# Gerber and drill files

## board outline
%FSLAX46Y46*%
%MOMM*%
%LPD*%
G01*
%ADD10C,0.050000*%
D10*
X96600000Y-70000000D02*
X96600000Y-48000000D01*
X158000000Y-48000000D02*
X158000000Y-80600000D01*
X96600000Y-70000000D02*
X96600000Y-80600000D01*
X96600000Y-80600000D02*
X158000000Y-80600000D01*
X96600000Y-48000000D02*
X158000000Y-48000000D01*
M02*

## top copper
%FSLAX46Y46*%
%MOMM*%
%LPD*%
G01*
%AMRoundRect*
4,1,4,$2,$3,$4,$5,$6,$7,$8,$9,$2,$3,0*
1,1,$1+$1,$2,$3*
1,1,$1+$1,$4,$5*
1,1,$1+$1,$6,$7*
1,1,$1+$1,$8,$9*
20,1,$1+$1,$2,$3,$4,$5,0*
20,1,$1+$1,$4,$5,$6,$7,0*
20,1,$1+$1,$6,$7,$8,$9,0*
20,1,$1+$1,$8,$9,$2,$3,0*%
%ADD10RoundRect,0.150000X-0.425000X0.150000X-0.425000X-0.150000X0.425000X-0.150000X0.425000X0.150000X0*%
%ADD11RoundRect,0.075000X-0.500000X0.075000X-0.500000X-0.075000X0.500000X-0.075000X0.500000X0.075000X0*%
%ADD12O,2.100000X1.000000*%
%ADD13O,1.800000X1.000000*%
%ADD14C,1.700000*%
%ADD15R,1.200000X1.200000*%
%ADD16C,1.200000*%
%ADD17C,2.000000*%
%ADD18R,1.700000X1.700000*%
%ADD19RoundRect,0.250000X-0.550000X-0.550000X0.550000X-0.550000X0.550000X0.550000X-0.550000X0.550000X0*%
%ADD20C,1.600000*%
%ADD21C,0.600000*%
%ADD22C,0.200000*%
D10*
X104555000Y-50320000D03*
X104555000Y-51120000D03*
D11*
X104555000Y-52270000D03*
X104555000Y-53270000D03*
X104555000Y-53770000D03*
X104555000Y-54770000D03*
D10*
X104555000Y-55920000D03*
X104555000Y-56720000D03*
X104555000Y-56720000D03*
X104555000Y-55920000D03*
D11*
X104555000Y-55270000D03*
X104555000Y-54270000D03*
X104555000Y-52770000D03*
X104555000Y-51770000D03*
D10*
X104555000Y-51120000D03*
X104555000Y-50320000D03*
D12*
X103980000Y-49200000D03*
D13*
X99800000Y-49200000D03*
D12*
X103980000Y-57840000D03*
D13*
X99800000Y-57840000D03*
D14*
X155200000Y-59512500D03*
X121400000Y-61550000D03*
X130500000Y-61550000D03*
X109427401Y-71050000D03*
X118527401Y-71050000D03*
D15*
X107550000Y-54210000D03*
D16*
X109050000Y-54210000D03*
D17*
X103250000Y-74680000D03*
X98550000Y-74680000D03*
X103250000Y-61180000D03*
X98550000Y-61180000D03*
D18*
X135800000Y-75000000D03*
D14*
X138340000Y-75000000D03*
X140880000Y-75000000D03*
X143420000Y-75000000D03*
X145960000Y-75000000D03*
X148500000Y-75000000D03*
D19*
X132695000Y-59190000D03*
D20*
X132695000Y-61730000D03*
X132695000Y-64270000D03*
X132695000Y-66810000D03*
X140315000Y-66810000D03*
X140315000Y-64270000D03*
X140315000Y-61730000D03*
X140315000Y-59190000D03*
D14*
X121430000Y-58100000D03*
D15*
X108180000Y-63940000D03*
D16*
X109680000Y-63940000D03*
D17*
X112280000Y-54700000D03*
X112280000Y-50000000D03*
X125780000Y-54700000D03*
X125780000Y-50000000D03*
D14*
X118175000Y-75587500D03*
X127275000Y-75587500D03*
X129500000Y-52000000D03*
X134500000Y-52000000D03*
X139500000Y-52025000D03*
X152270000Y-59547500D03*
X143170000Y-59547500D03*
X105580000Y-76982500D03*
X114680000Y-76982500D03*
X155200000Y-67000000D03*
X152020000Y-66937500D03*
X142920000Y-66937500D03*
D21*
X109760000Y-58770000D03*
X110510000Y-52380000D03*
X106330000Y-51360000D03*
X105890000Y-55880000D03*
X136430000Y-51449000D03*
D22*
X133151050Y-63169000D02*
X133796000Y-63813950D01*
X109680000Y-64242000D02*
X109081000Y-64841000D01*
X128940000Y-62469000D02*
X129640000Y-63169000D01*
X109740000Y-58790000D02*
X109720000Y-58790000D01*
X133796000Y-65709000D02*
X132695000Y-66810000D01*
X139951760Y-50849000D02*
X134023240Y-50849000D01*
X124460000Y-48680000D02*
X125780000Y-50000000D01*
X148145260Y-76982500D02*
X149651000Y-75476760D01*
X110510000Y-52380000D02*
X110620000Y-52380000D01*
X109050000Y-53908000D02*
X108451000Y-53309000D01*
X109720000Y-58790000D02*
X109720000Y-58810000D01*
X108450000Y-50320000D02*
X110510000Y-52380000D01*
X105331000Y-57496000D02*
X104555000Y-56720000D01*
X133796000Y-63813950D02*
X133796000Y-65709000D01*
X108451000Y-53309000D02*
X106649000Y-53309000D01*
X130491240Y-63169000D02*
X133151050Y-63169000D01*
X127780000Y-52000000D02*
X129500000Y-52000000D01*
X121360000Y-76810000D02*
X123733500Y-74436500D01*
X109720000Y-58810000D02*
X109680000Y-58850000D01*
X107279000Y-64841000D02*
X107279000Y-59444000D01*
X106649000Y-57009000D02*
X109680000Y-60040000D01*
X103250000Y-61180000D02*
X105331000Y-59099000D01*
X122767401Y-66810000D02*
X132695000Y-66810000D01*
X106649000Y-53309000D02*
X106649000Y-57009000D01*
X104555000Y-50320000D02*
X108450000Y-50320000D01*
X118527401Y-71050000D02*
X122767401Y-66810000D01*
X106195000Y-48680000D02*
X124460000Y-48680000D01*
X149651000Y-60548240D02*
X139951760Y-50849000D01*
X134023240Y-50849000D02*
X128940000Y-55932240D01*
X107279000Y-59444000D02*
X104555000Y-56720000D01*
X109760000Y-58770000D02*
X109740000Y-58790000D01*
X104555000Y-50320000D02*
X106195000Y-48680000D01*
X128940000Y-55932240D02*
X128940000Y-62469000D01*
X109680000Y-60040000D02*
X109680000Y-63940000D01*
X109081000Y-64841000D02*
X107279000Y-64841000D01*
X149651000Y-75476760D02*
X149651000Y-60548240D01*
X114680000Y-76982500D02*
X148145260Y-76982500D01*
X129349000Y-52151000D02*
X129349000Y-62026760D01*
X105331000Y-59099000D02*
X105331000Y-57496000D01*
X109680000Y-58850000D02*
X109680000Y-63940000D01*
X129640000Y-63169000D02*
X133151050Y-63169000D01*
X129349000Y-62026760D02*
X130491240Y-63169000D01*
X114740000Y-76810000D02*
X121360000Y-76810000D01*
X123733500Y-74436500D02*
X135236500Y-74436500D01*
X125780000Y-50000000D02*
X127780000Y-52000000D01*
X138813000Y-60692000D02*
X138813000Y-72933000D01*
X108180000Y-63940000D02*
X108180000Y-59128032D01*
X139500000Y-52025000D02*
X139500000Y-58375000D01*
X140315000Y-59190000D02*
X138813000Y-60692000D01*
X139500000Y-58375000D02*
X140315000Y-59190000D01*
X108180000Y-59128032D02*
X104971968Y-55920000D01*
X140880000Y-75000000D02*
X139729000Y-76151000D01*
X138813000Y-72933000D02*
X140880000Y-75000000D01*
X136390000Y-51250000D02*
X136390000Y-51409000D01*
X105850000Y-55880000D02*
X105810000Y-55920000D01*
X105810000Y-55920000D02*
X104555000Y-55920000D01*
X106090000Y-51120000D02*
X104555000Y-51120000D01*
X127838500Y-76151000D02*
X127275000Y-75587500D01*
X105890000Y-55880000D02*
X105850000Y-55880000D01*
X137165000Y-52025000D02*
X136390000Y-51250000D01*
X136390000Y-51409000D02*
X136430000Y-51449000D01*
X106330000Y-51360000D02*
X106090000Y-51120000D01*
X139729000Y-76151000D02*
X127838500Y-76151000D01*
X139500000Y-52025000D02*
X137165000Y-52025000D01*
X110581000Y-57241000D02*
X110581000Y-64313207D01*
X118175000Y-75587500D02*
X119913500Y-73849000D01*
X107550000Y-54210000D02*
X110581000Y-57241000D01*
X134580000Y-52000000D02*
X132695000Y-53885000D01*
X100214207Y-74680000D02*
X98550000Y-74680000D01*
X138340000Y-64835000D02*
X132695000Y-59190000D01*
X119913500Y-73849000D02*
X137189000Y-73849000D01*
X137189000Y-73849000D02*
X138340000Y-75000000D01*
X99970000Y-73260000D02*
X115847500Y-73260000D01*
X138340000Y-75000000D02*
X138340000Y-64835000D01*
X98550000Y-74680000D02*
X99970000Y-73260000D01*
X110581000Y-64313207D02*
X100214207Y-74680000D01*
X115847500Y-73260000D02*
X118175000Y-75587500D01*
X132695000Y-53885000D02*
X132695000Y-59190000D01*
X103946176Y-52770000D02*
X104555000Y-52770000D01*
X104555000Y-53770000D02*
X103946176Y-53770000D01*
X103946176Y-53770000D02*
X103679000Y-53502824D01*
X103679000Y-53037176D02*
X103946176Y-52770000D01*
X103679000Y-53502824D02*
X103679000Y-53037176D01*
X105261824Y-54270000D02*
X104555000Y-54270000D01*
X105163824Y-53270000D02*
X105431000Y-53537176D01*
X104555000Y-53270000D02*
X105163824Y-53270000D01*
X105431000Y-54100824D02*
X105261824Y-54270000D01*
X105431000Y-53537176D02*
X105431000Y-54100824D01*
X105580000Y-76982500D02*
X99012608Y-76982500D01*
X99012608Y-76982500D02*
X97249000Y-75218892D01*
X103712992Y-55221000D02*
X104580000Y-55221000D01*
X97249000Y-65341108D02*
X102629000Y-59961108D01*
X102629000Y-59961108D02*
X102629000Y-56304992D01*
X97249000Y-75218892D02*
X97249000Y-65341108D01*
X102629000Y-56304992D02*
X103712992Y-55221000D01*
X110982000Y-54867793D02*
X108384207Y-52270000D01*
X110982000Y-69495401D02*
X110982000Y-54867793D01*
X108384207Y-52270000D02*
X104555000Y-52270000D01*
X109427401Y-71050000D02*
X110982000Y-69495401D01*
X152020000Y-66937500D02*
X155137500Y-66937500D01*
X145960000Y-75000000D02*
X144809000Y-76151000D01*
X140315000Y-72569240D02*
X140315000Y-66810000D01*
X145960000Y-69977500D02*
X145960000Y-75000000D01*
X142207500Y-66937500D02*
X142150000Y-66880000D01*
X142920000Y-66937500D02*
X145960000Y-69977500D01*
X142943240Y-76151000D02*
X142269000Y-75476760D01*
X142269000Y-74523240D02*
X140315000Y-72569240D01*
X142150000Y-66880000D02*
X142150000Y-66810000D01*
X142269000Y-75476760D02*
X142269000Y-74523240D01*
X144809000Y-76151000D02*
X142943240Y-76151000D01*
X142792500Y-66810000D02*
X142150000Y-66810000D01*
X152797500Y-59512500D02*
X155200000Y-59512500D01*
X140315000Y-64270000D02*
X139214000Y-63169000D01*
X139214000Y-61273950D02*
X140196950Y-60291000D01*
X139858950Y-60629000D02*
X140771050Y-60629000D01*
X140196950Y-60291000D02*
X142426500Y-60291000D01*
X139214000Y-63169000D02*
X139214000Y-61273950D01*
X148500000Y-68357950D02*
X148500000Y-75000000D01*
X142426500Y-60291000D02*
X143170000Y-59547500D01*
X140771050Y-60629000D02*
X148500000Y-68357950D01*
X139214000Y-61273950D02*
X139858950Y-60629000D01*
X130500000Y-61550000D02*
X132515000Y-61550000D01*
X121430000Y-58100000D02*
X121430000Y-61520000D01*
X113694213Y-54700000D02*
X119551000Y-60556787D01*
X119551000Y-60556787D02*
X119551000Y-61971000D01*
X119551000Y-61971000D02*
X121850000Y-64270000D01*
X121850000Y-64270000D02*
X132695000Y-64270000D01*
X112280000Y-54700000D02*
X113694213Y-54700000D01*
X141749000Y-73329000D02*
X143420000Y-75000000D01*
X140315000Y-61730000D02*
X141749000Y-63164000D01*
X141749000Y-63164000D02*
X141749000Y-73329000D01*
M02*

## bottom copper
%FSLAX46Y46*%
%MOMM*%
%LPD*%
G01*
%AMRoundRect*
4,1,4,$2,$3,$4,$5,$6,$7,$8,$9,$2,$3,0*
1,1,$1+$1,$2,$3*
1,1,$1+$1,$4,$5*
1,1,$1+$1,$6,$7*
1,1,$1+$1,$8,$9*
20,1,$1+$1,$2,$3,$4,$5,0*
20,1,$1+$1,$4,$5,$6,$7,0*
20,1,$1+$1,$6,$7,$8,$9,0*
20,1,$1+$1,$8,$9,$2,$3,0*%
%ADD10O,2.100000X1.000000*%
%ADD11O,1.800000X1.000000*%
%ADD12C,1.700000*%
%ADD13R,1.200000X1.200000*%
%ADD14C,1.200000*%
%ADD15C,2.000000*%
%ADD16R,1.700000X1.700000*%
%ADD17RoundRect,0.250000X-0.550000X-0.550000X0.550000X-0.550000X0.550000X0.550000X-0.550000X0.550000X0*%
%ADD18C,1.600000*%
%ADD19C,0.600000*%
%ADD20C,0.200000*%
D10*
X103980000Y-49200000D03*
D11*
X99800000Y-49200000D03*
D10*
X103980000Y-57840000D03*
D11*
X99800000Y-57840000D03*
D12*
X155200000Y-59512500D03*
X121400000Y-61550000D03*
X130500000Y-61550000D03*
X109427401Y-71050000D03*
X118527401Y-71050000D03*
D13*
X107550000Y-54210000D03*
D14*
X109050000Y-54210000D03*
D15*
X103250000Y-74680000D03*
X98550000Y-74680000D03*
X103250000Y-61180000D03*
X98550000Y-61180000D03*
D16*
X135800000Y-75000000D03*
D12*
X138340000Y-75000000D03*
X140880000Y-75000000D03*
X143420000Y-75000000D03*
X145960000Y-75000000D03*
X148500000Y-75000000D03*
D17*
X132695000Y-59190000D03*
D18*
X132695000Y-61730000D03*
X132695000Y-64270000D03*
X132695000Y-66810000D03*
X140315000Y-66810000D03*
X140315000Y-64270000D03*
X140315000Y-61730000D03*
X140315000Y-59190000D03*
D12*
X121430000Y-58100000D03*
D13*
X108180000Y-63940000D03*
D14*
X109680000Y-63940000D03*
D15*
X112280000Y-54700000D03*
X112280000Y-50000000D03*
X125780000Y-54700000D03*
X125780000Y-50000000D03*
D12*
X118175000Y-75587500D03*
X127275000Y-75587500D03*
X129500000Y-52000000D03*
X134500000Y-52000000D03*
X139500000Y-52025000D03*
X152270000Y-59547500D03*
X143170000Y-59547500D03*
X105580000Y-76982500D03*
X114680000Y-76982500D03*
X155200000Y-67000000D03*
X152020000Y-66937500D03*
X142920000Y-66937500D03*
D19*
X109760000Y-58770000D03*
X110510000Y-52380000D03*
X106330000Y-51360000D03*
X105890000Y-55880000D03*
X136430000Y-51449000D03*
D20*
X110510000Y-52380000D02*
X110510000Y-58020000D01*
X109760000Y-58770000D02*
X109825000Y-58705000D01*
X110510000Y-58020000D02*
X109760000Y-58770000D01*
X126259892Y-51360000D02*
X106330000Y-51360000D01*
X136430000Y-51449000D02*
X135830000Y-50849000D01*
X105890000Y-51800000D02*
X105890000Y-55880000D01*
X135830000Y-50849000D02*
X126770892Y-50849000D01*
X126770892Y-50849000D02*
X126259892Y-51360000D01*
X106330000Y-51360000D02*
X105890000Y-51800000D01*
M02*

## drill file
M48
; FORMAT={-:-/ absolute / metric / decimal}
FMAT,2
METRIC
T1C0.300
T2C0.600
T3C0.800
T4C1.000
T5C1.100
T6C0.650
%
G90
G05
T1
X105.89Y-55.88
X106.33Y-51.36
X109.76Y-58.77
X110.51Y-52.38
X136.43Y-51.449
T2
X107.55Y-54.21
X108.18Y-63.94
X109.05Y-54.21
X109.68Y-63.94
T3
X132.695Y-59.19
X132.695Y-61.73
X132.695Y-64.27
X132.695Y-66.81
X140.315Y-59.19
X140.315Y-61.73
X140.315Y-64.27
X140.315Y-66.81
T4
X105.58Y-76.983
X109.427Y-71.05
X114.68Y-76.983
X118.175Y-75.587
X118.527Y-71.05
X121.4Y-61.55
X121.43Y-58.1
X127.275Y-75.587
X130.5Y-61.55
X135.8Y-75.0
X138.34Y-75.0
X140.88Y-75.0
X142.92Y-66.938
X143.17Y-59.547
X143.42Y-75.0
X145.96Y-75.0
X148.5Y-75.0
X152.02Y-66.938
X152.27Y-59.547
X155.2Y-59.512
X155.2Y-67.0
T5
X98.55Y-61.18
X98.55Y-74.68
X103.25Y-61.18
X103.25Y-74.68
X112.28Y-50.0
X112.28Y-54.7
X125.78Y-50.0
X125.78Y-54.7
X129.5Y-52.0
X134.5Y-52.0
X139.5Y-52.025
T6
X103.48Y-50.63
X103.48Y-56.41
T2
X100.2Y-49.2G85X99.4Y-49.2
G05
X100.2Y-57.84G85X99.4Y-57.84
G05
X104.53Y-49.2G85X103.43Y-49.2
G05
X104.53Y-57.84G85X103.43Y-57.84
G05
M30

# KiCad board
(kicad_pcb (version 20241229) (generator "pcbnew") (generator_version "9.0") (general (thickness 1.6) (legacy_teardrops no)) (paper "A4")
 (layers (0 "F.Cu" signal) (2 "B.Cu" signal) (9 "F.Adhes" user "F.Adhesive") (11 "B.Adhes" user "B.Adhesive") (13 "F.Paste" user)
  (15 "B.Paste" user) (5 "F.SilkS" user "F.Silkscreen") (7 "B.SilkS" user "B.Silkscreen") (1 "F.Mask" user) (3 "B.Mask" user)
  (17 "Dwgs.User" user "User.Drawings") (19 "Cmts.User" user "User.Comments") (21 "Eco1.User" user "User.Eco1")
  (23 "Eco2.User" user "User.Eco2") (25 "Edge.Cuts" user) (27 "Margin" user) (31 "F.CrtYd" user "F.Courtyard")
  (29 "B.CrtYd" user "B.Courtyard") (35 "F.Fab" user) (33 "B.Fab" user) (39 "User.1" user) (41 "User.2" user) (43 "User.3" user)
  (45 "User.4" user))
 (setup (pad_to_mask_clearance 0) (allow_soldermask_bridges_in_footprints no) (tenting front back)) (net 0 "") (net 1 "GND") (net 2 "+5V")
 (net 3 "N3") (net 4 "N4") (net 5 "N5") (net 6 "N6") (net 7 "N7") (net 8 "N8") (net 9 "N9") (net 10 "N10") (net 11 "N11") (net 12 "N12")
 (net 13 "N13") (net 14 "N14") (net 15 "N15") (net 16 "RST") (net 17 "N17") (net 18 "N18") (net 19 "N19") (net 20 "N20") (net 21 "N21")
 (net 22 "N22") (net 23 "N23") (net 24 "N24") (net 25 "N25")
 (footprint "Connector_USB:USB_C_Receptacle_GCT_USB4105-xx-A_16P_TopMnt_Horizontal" (layer "F.Cu") (at 100.875 53.52 -90)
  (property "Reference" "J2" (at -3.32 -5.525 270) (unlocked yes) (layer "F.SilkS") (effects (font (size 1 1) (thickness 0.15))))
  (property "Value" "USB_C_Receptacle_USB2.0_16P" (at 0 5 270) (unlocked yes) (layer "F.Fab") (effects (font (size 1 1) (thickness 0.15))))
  (pad "" np_thru_hole circle (at -2.89 -2.605 270) (size 0.65 0.65) (drill 0.65) (layers "*.Cu" "*.Mask"))
  (pad "" np_thru_hole circle (at 2.89 -2.605 270) (size 0.65 0.65) (drill 0.65) (layers "*.Cu" "*.Mask"))
  (pad "A1" smd roundrect (at -3.2 -3.68 270) (size 0.6 1.15) (layers "F.Cu" "F.Mask" "F.Paste") (roundrect_rratio 0.25) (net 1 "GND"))
  (pad "A4" smd roundrect (at -2.4 -3.68 270) (size 0.6 1.15) (layers "F.Cu" "F.Mask" "F.Paste") (roundrect_rratio 0.25) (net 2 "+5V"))
  (pad "A5" smd roundrect (at -1.25 -3.68 270) (size 0.3 1.15) (layers "F.Cu" "F.Mask" "F.Paste") (roundrect_rratio 0.25) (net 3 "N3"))
  (pad "A6" smd roundrect (at -0.25 -3.68 270) (size 0.3 1.15) (layers "F.Cu" "F.Mask" "F.Paste") (roundrect_rratio 0.25) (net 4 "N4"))
  (pad "A7" smd roundrect (at 0.25 -3.68 270) (size 0.3 1.15) (layers "F.Cu" "F.Mask" "F.Paste") (roundrect_rratio 0.25) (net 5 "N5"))
  (pad "A8" smd roundrect (at 1.25 -3.68 270) (size 0.3 1.15) (layers "F.Cu" "F.Mask" "F.Paste") (roundrect_rratio 0.25) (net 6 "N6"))
  (pad "A9" smd roundrect (at 2.4 -3.68 270) (size 0.6 1.15) (layers "F.Cu" "F.Mask" "F.Paste") (roundrect_rratio 0.25) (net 2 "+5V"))
  (pad "A12" smd roundrect (at 3.2 -3.68 270) (size 0.6 1.15) (layers "F.Cu" "F.Mask" "F.Paste") (roundrect_rratio 0.25) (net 1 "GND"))
  (pad "B1" smd roundrect (at 3.2 -3.68 270) (size 0.6 1.15) (layers "F.Cu" "F.Mask" "F.Paste") (roundrect_rratio 0.25) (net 1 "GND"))
  (pad "B4" smd roundrect (at 2.4 -3.68 270) (size 0.6 1.15) (layers "F.Cu" "F.Mask" "F.Paste") (roundrect_rratio 0.25) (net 2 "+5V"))
  (pad "B5" smd roundrect (at 1.75 -3.68 270) (size 0.3 1.15) (layers "F.Cu" "F.Mask" "F.Paste") (roundrect_rratio 0.25) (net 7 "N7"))
  (pad "B6" smd roundrect (at 0.75 -3.68 270) (size 0.3 1.15) (layers "F.Cu" "F.Mask" "F.Paste") (roundrect_rratio 0.25) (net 4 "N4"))
  (pad "B7" smd roundrect (at -0.75 -3.68 270) (size 0.3 1.15) (layers "F.Cu" "F.Mask" "F.Paste") (roundrect_rratio 0.25) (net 5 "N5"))
  (pad "B8" smd roundrect (at -1.75 -3.68 270) (size 0.3 1.15) (layers "F.Cu" "F.Mask" "F.Paste") (roundrect_rratio 0.25) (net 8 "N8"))
  (pad "B9" smd roundrect (at -2.4 -3.68 270) (size 0.6 1.15) (layers "F.Cu" "F.Mask" "F.Paste") (roundrect_rratio 0.25) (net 2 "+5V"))
  (pad "B12" smd roundrect (at -3.2 -3.68 270) (size 0.6 1.15) (layers "F.Cu" "F.Mask" "F.Paste") (roundrect_rratio 0.25) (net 1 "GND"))
  (pad "S1" thru_hole oval (at -4.32 -3.105 270) (size 1 2.1) (drill oval 0.6 1.7) (layers "*.Cu" "*.Mask" "F.Paste")
   (remove_unused_layers no) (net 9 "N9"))
  (pad "S1" thru_hole oval (at -4.32 1.075 270) (size 1 1.8) (drill oval 0.6 1.4) (layers "*.Cu" "*.Mask" "F.Paste")
   (remove_unused_layers no) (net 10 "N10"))
  (pad "S1" thru_hole oval (at 4.32 -3.105 270) (size 1 2.1) (drill oval 0.6 1.7) (layers "*.Cu" "*.Mask" "F.Paste")
   (remove_unused_layers no) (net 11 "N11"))
  (pad "S1" thru_hole oval (at 4.32 1.075 270) (size 1 1.8) (drill oval 0.6 1.4) (layers "*.Cu" "*.Mask" "F.Paste")
   (remove_unused_layers no) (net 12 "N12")))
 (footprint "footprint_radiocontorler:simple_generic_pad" (layer "F.Cu") (at 155.2 54.0125)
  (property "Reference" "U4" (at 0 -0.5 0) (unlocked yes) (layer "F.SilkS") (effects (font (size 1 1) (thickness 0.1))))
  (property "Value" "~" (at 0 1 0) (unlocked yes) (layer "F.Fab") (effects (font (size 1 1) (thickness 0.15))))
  (pad "1" thru_hole circle (at 0 5.5) (size 1.7 1.7) (drill 1) (layers "*.Cu" "*.Mask") (remove_unused_layers no) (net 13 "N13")))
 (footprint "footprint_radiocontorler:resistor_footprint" (layer "F.Cu") (at 126.2 57.15)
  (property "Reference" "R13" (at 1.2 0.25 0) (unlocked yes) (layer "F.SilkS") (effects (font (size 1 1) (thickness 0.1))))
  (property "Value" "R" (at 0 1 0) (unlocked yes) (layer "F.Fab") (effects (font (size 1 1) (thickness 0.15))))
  (pad "1" thru_hole circle (at -4.8 4.4) (size 1.7 1.7) (drill 1) (layers "*.Cu" "*.Mask") (remove_unused_layers no) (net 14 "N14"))
  (pad "2" thru_hole circle (at 4.3 4.4) (size 1.7 1.7) (drill 1) (layers "*.Cu" "*.Mask") (remove_unused_layers no) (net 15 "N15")))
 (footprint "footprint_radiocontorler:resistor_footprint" (layer "F.Cu") (at 114.227401 66.65)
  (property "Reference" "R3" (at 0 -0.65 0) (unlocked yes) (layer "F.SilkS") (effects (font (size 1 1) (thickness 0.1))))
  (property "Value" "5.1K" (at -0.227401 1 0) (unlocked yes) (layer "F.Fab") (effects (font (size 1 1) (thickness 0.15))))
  (pad "1" thru_hole circle (at -4.8 4.4) (size 1.7 1.7) (drill 1) (layers "*.Cu" "*.Mask") (remove_unused_layers no) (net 3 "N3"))
  (pad "2" thru_hole circle (at 4.3 4.4) (size 1.7 1.7) (drill 1) (layers "*.Cu" "*.Mask") (remove_unused_layers no) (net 1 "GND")))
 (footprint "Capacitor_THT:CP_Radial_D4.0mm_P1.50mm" (layer "F.Cu") (at 107.55 54.21)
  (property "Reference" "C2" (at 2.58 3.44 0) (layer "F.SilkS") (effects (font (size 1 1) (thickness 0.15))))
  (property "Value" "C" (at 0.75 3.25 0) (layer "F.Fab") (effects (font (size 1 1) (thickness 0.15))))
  (pad "1" thru_hole rect (at 0 0) (size 1.2 1.2) (drill 0.6) (layers "*.Cu" "*.Mask") (remove_unused_layers no) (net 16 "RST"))
  (pad "2" thru_hole circle (at 1.5 0) (size 1.2 1.2) (drill 0.6) (layers "*.Cu" "*.Mask") (remove_unused_layers no) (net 1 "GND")))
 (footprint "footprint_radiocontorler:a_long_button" (layer "F.Cu") (at 100.85 67.88 180)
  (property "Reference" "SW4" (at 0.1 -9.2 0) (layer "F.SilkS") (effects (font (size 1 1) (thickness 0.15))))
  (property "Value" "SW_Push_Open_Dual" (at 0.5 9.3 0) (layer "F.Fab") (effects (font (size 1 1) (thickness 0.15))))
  (pad "1" thru_hole circle (at -2.4 -6.8 270) (size 2 2) (drill 1.1) (layers "*.Cu" "*.Mask") (remove_unused_layers no) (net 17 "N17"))
  (pad "2" thru_hole circle (at 2.3 -6.8 270) (size 2 2) (drill 1.1) (layers "*.Cu" "*.Mask") (remove_unused_layers no) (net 16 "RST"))
  (pad "3" thru_hole circle (at -2.4 6.7 270) (size 2 2) (drill 1.1) (layers "*.Cu" "*.Mask") (remove_unused_layers no) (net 1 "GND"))
  (pad "4" thru_hole circle (at 2.3 6.7 270) (size 2 2) (drill 1.1) (layers "*.Cu" "*.Mask") (remove_unused_layers no) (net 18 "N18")))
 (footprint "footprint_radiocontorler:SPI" (layer "F.Cu") (at 130.96 75 90)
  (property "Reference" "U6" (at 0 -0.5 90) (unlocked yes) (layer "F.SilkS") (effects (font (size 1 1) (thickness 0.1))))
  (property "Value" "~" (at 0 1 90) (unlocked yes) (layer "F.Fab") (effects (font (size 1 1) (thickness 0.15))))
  (pad "1" thru_hole rect (at 0 4.84 90) (size 1.7 1.7) (drill 1) (layers "*.Cu" "*.Mask") (remove_unused_layers no) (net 1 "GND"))
  (pad "2" thru_hole circle (at 0 7.38 90) (size 1.7 1.7) (drill 1) (layers "*.Cu" "*.Mask") (remove_unused_layers no) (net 16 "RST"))
  (pad "3" thru_hole circle (at 0 9.92 90) (size 1.7 1.7) (drill 1) (layers "*.Cu" "*.Mask") (remove_unused_layers no) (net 2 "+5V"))
  (pad "4" thru_hole circle (at 0 12.46 90) (size 1.7 1.7) (drill 1) (layers "*.Cu" "*.Mask") (remove_unused_layers no) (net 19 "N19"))
  (pad "5" thru_hole circle (at 0 15 90) (size 1.7 1.7) (drill 1) (layers "*.Cu" "*.Mask") (remove_unused_layers no) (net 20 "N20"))
  (pad "6" thru_hole circle (at 0 17.54 90) (size 1.7 1.7) (drill 1) (layers "*.Cu" "*.Mask") (remove_unused_layers no) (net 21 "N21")))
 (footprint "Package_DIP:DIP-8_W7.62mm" (layer "F.Cu") (at 132.695 59.19)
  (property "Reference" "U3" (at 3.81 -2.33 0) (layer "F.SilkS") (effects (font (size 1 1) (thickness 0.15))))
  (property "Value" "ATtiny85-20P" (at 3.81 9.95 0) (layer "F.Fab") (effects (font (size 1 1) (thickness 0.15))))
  (pad "1" thru_hole roundrect (at 0 0) (size 1.6 1.6) (drill 0.8) (layers "*.Cu" "*.Mask") (remove_unused_layers no)
   (roundrect_rratio 0.15625) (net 16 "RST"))
  (pad "2" thru_hole circle (at 0 2.54) (size 1.6 1.6) (drill 0.8) (layers "*.Cu" "*.Mask") (remove_unused_layers no) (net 15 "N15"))
  (pad "3" thru_hole circle (at 0 5.08) (size 1.6 1.6) (drill 0.8) (layers "*.Cu" "*.Mask") (remove_unused_layers no) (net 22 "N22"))
  (pad "4" thru_hole circle (at 0 7.62) (size 1.6 1.6) (drill 0.8) (layers "*.Cu" "*.Mask") (remove_unused_layers no) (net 1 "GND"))
  (pad "5" thru_hole circle (at 7.62 7.62) (size 1.6 1.6) (drill 0.8) (layers "*.Cu" "*.Mask") (remove_unused_layers no) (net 20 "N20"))
  (pad "6" thru_hole circle (at 7.62 5.08) (size 1.6 1.6) (drill 0.8) (layers "*.Cu" "*.Mask") (remove_unused_layers no) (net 21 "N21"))
  (pad "7" thru_hole circle (at 7.62 2.54) (size 1.6 1.6) (drill 0.8) (layers "*.Cu" "*.Mask") (remove_unused_layers no) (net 19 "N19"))
  (pad "8" thru_hole circle (at 7.62 0) (size 1.6 1.6) (drill 0.8) (layers "*.Cu" "*.Mask") (remove_unused_layers no) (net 2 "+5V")))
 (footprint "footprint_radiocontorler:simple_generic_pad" (layer "F.Cu") (at 121.43 52.6)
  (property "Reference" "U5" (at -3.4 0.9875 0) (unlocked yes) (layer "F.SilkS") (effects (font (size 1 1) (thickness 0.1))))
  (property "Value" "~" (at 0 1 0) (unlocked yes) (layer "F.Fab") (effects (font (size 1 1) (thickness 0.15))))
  (pad "1" thru_hole circle (at 0 5.5) (size 1.7 1.7) (drill 1) (layers "*.Cu" "*.Mask") (remove_unused_layers no) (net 14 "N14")))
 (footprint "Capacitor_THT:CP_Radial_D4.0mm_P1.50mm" (layer "F.Cu") (at 108.18 63.94)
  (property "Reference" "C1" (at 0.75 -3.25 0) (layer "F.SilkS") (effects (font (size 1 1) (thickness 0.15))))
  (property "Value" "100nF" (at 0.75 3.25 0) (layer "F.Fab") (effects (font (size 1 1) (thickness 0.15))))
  (pad "1" thru_hole rect (at 0 0) (size 1.2 1.2) (drill 0.6) (layers "*.Cu" "*.Mask") (remove_unused_layers no) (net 2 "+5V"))
  (pad "2" thru_hole circle (at 1.5 0) (size 1.2 1.2) (drill 0.6) (layers "*.Cu" "*.Mask") (remove_unused_layers no) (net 1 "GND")))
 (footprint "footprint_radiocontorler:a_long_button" (layer "F.Cu") (at 119.08 52.3 90)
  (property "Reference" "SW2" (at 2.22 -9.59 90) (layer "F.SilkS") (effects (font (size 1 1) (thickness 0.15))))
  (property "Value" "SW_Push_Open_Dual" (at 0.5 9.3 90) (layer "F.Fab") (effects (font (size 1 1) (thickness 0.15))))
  (pad "1" thru_hole circle (at -2.4 -6.8 180) (size 2 2) (drill 1.1) (layers "*.Cu" "*.Mask") (remove_unused_layers no) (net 22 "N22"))
  (pad "2" thru_hole circle (at 2.3 -6.8 180) (size 2 2) (drill 1.1) (layers "*.Cu" "*.Mask") (remove_unused_layers no) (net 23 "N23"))
  (pad "3" thru_hole circle (at -2.4 6.7 180) (size 2 2) (drill 1.1) (layers "*.Cu" "*.Mask") (remove_unused_layers no) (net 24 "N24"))
  (pad "4" thru_hole circle (at 2.3 6.7 180) (size 2 2) (drill 1.1) (layers "*.Cu" "*.Mask") (remove_unused_layers no) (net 1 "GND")))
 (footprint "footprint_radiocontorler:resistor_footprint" (layer "F.Cu") (at 122.975 71.1875)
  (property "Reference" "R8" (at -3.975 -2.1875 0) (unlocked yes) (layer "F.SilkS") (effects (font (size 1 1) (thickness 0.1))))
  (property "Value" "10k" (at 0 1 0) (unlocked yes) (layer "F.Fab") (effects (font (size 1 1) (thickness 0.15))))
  (pad "1" thru_hole circle (at -4.8 4.4) (size 1.7 1.7) (drill 1) (layers "*.Cu" "*.Mask") (remove_unused_layers no) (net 16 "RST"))
  (pad "2" thru_hole circle (at 4.3 4.4) (size 1.7 1.7) (drill 1) (layers "*.Cu" "*.Mask") (remove_unused_layers no) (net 2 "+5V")))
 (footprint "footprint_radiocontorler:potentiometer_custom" (layer "F.Cu") (at 125.4 51.75 90)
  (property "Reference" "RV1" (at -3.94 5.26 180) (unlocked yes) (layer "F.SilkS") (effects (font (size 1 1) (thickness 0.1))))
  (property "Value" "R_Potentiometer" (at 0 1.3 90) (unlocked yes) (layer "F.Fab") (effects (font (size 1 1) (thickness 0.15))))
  (pad "1" thru_hole circle (at -0.25 4.1 90) (size 1.7 1.7) (drill 1.1) (layers "*.Cu" "*.Mask") (remove_unused_layers no) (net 1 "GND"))
  (pad "2" thru_hole circle (at -0.25 9.1 90) (size 1.7 1.7) (drill 1.1) (layers "*.Cu" "*.Mask") (remove_unused_layers no) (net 16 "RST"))
  (pad "3" thru_hole circle (at -0.275 14.1 90) (size 1.7 1.7) (drill 1.1) (layers "*.Cu" "*.Mask") (remove_unused_layers no) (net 2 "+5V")))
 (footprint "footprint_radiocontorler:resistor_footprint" (layer "F.Cu") (at 147.47 63.9475 180)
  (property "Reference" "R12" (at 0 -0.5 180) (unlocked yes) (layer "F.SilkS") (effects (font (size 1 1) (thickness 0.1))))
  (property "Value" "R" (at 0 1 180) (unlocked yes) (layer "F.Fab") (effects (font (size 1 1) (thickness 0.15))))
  (pad "1" thru_hole circle (at -4.8 4.4 180) (size 1.7 1.7) (drill 1) (layers "*.Cu" "*.Mask") (remove_unused_layers no) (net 13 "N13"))
  (pad "2" thru_hole circle (at 4.3 4.4 180) (size 1.7 1.7) (drill 1) (layers "*.Cu" "*.Mask") (remove_unused_layers no) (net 21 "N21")))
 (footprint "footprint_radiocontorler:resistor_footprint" (layer "F.Cu") (at 110.38 72.5825)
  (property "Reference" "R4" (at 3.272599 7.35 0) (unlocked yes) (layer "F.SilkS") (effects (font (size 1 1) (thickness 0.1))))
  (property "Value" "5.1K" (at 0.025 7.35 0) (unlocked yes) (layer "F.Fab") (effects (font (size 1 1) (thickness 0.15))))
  (pad "1" thru_hole circle (at -4.8 4.4) (size 1.7 1.7) (drill 1) (layers "*.Cu" "*.Mask") (remove_unused_layers no) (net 7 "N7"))
  (pad "2" thru_hole circle (at 4.3 4.4) (size 1.7 1.7) (drill 1) (layers "*.Cu" "*.Mask") (remove_unused_layers no) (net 1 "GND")))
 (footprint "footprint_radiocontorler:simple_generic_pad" (layer "F.Cu") (at 155.2 61.5)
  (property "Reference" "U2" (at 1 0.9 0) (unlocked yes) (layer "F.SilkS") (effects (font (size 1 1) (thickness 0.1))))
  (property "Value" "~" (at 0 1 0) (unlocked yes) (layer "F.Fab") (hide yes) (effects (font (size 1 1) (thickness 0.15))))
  (pad "1" thru_hole circle (at 0 5.5) (size 1.7 1.7) (drill 1) (layers "*.Cu" "*.Mask") (remove_unused_layers no) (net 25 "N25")))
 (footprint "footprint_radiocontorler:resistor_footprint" (layer "F.Cu") (at 147.22 71.3375 180)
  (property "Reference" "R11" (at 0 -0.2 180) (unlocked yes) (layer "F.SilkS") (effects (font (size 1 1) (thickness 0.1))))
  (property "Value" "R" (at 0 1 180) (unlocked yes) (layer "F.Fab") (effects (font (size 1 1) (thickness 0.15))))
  (pad "1" thru_hole circle (at -4.8 4.4 180) (size 1.7 1.7) (drill 1) (layers "*.Cu" "*.Mask") (remove_unused_layers no) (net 25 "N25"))
  (pad "2" thru_hole circle (at 4.3 4.4 180) (size 1.7 1.7) (drill 1) (layers "*.Cu" "*.Mask") (remove_unused_layers no) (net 20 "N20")))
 (gr_line (start 96.6 70) (end 96.6 48) (stroke (width 0.05) (type default)) (layer "Edge.Cuts"))
 (gr_line (start 158 48) (end 158 80.6) (stroke (width 0.05) (type default)) (layer "Edge.Cuts"))
 (gr_line (start 96.6 70) (end 96.6 80.6) (stroke (width 0.05) (type default)) (layer "Edge.Cuts"))
 (gr_line (start 96.6 80.6) (end 158 80.6) (stroke (width 0.05) (type default)) (layer "Edge.Cuts"))
 (gr_line (start 96.6 48) (end 158 48) (stroke (width 0.05) (type default)) (layer "Edge.Cuts"))
 (segment (start 133.15105 63.169) (end 133.796 63.81395) (width 0.2) (layer "F.Cu") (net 1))
 (segment (start 109.68 64.242) (end 109.081 64.841) (width 0.2) (layer "F.Cu") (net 1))
 (segment (start 128.94 62.469) (end 129.64 63.169) (width 0.2) (layer "F.Cu") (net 1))
 (segment (start 109.74 58.79) (end 109.72 58.79) (width 0.2) (layer "F.Cu") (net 1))
 (segment (start 133.796 65.709) (end 132.695 66.81) (width 0.2) (layer "F.Cu") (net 1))
 (segment (start 139.95176 50.849) (end 134.02324 50.849) (width 0.2) (layer "F.Cu") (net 1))
 (segment (start 124.46 48.68) (end 125.78 50) (width 0.2) (layer "F.Cu") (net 1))
 (segment (start 148.14526 76.9825) (end 149.651 75.47676) (width 0.2) (layer "F.Cu") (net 1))
 (segment (start 110.51 52.38) (end 110.62 52.38) (width 0.2) (layer "F.Cu") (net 1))
 (segment (start 109.05 53.908) (end 108.451 53.309) (width 0.2) (layer "F.Cu") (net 1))
 (segment (start 109.72 58.79) (end 109.72 58.81) (width 0.2) (layer "F.Cu") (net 1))
 (segment (start 108.45 50.32) (end 110.51 52.38) (width 0.2) (layer "F.Cu") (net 1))
 (segment (start 105.331 57.496) (end 104.555 56.72) (width 0.2) (layer "F.Cu") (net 1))
 (segment (start 133.796 63.81395) (end 133.796 65.709) (width 0.2) (layer "F.Cu") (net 1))
 (segment (start 108.451 53.309) (end 106.649 53.309) (width 0.2) (layer "F.Cu") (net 1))
 (segment (start 130.49124 63.169) (end 133.15105 63.169) (width 0.2) (layer "F.Cu") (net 1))
 (segment (start 127.78 52) (end 129.5 52) (width 0.2) (layer "F.Cu") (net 1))
 (segment (start 121.36 76.81) (end 123.7335 74.4365) (width 0.2) (layer "F.Cu") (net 1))
 (segment (start 109.72 58.81) (end 109.68 58.85) (width 0.2) (layer "F.Cu") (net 1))
 (segment (start 107.279 64.841) (end 107.279 59.444) (width 0.2) (layer "F.Cu") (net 1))
 (segment (start 106.649 57.009) (end 109.68 60.04) (width 0.2) (layer "F.Cu") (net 1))
 (segment (start 103.25 61.18) (end 105.331 59.099) (width 0.2) (layer "F.Cu") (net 1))
 (segment (start 122.767401 66.81) (end 132.695 66.81) (width 0.2) (layer "F.Cu") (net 1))
 (segment (start 106.649 53.309) (end 106.649 57.009) (width 0.2) (layer "F.Cu") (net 1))
 (segment (start 104.555 50.32) (end 108.45 50.32) (width 0.2) (layer "F.Cu") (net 1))
 (segment (start 118.527401 71.05) (end 122.767401 66.81) (width 0.2) (layer "F.Cu") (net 1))
 (segment (start 106.195 48.68) (end 124.46 48.68) (width 0.2) (layer "F.Cu") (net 1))
 (segment (start 149.651 60.54824) (end 139.95176 50.849) (width 0.2) (layer "F.Cu") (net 1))
 (segment (start 134.02324 50.849) (end 128.94 55.93224) (width 0.2) (layer "F.Cu") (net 1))
 (segment (start 107.279 59.444) (end 104.555 56.72) (width 0.2) (layer "F.Cu") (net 1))
 (segment (start 109.76 58.77) (end 109.74 58.79) (width 0.2) (layer "F.Cu") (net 1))
 (segment (start 104.555 50.32) (end 106.195 48.68) (width 0.2) (layer "F.Cu") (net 1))
 (segment (start 128.94 55.93224) (end 128.94 62.469) (width 0.2) (layer "F.Cu") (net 1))
 (segment (start 109.68 60.04) (end 109.68 63.94) (width 0.2) (layer "F.Cu") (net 1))
 (segment (start 109.081 64.841) (end 107.279 64.841) (width 0.2) (layer "F.Cu") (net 1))
 (segment (start 149.651 75.47676) (end 149.651 60.54824) (width 0.2) (layer "F.Cu") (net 1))
 (segment (start 114.68 76.9825) (end 148.14526 76.9825) (width 0.2) (layer "F.Cu") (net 1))
 (segment (start 129.349 52.151) (end 129.349 62.02676) (width 0.2) (layer "F.Cu") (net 1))
 (segment (start 105.331 59.099) (end 105.331 57.496) (width 0.2) (layer "F.Cu") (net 1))
 (segment (start 109.68 58.85) (end 109.68 63.94) (width 0.2) (layer "F.Cu") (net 1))
 (segment (start 129.64 63.169) (end 133.15105 63.169) (width 0.2) (layer "F.Cu") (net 1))
 (segment (start 129.349 62.02676) (end 130.49124 63.169) (width 0.2) (layer "F.Cu") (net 1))
 (segment (start 114.74 76.81) (end 121.36 76.81) (width 0.2) (layer "F.Cu") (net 1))
 (segment (start 123.7335 74.4365) (end 135.2365 74.4365) (width 0.2) (layer "F.Cu") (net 1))
 (segment (start 125.78 50) (end 127.78 52) (width 0.2) (layer "F.Cu") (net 1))
 (via (at 109.76 58.77) (size 0.6) (drill 0.3) (layers "F.Cu" "B.Cu") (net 1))
 (via (at 110.51 52.38) (size 0.6) (drill 0.3) (layers "F.Cu" "B.Cu") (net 1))
 (segment (start 110.51 52.38) (end 110.51 58.02) (width 0.2) (layer "B.Cu") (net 1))
 (segment (start 109.76 58.77) (end 109.825 58.705) (width 0.2) (layer "B.Cu") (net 1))
 (segment (start 110.51 58.02) (end 109.76 58.77) (width 0.2) (layer "B.Cu") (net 1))
 (segment (start 138.813 60.692) (end 138.813 72.933) (width 0.2) (layer "F.Cu") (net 2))
 (segment (start 108.18 63.94) (end 108.18 59.128032) (width 0.2) (layer "F.Cu") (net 2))
 (segment (start 139.5 52.025) (end 139.5 58.375) (width 0.2) (layer "F.Cu") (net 2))
 (segment (start 140.315 59.19) (end 138.813 60.692) (width 0.2) (layer "F.Cu") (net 2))
 (segment (start 139.5 58.375) (end 140.315 59.19) (width 0.2) (layer "F.Cu") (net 2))
 (segment (start 108.18 59.128032) (end 104.971968 55.92) (width 0.2) (layer "F.Cu") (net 2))
 (segment (start 140.88 75) (end 139.729 76.151) (width 0.2) (layer "F.Cu") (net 2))
 (segment (start 138.813 72.933) (end 140.88 75) (width 0.2) (layer "F.Cu") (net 2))
 (segment (start 136.39 51.25) (end 136.39 51.409) (width 0.2) (layer "F.Cu") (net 2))
 (segment (start 105.85 55.88) (end 105.81 55.92) (width 0.2) (layer "F.Cu") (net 2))
 (segment (start 105.81 55.92) (end 104.555 55.92) (width 0.2) (layer "F.Cu") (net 2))
 (segment (start 106.09 51.12) (end 104.555 51.12) (width 0.2) (layer "F.Cu") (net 2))
 (segment (start 127.8385 76.151) (end 127.275 75.5875) (width 0.2) (layer "F.Cu") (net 2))
 (segment (start 105.89 55.88) (end 105.85 55.88) (width 0.2) (layer "F.Cu") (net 2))
 (segment (start 137.165 52.025) (end 136.39 51.25) (width 0.2) (layer "F.Cu") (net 2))
 (segment (start 136.39 51.409) (end 136.43 51.449) (width 0.2) (layer "F.Cu") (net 2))
 (segment (start 106.33 51.36) (end 106.09 51.12) (width 0.2) (layer "F.Cu") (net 2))
 (segment (start 139.729 76.151) (end 127.8385 76.151) (width 0.2) (layer "F.Cu") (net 2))
 (segment (start 139.5 52.025) (end 137.165 52.025) (width 0.2) (layer "F.Cu") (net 2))
 (via (at 106.33 51.36) (size 0.6) (drill 0.3) (layers "F.Cu" "B.Cu") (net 2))
 (via (at 105.89 55.88) (size 0.6) (drill 0.3) (layers "F.Cu" "B.Cu") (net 2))
 (via (at 136.43 51.449) (size 0.6) (drill 0.3) (layers "F.Cu" "B.Cu") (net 2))
 (segment (start 126.259892 51.36) (end 106.33 51.36) (width 0.2) (layer "B.Cu") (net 2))
 (segment (start 136.43 51.449) (end 135.83 50.849) (width 0.2) (layer "B.Cu") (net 2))
 (segment (start 105.89 51.8) (end 105.89 55.88) (width 0.2) (layer "B.Cu") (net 2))
 (segment (start 135.83 50.849) (end 126.770892 50.849) (width 0.2) (layer "B.Cu") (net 2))
 (segment (start 126.770892 50.849) (end 126.259892 51.36) (width 0.2) (layer "B.Cu") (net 2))
 (segment (start 106.33 51.36) (end 105.89 51.8) (width 0.2) (layer "B.Cu") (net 2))
 (segment (start 110.581 57.241) (end 110.581 64.313207) (width 0.2) (layer "F.Cu") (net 16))
 (segment (start 118.175 75.5875) (end 119.9135 73.849) (width 0.2) (layer "F.Cu") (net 16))
 (segment (start 107.55 54.21) (end 110.581 57.241) (width 0.2) (layer "F.Cu") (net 16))
 (segment (start 134.58 52) (end 132.695 53.885) (width 0.2) (layer "F.Cu") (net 16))
 (segment (start 100.214207 74.68) (end 98.55 74.68) (width 0.2) (layer "F.Cu") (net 16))
 (segment (start 138.34 64.835) (end 132.695 59.19) (width 0.2) (layer "F.Cu") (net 16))
 (segment (start 119.9135 73.849) (end 137.189 73.849) (width 0.2) (layer "F.Cu") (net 16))
 (segment (start 137.189 73.849) (end 138.34 75) (width 0.2) (layer "F.Cu") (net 16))
 (segment (start 99.97 73.26) (end 115.8475 73.26) (width 0.2) (layer "F.Cu") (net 16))
 (segment (start 138.34 75) (end 138.34 64.835) (width 0.2) (layer "F.Cu") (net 16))
 (segment (start 98.55 74.68) (end 99.97 73.26) (width 0.2) (layer "F.Cu") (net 16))
 (segment (start 110.581 64.313207) (end 100.214207 74.68) (width 0.2) (layer "F.Cu") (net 16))
 (segment (start 115.8475 73.26) (end 118.175 75.5875) (width 0.2) (layer "F.Cu") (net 16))
 (segment (start 132.695 53.885) (end 132.695 59.19) (width 0.2) (layer "F.Cu") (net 16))
 (segment (start 103.946176 52.77) (end 104.555 52.77) (width 0.2) (layer "F.Cu") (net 5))
 (segment (start 104.555 53.77) (end 103.946176 53.77) (width 0.2) (layer "F.Cu") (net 5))
 (segment (start 103.946176 53.77) (end 103.679 53.502824) (width 0.2) (layer "F.Cu") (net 5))
 (segment (start 103.679 53.037176) (end 103.946176 52.77) (width 0.2) (layer "F.Cu") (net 5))
 (segment (start 103.679 53.502824) (end 103.679 53.037176) (width 0.2) (layer "F.Cu") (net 5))
 (segment (start 105.261824 54.27) (end 104.555 54.27) (width 0.2) (layer "F.Cu") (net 4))
 (segment (start 105.163824 53.27) (end 105.431 53.537176) (width 0.2) (layer "F.Cu") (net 4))
 (segment (start 104.555 53.27) (end 105.163824 53.27) (width 0.2) (layer "F.Cu") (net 4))
 (segment (start 105.431 54.100824) (end 105.261824 54.27) (width 0.2) (layer "F.Cu") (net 4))
 (segment (start 105.431 53.537176) (end 105.431 54.100824) (width 0.2) (layer "F.Cu") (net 4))
 (segment (start 105.58 76.9825) (end 99.012608 76.9825) (width 0.2) (layer "F.Cu") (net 7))
 (segment (start 99.012608 76.9825) (end 97.249 75.218892) (width 0.2) (layer "F.Cu") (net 7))
 (segment (start 103.712992 55.221) (end 104.58 55.221) (width 0.2) (layer "F.Cu") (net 7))
 (segment (start 97.249 65.341108) (end 102.629 59.961108) (width 0.2) (layer "F.Cu") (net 7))
 (segment (start 102.629 59.961108) (end 102.629 56.304992) (width 0.2) (layer "F.Cu") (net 7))
 (segment (start 97.249 75.218892) (end 97.249 65.341108) (width 0.2) (layer "F.Cu") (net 7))
 (segment (start 102.629 56.304992) (end 103.712992 55.221) (width 0.2) (layer "F.Cu") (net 7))
 (segment (start 110.982 54.867793) (end 108.384207 52.27) (width 0.2) (layer "F.Cu") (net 3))
 (segment (start 110.982 69.495401) (end 110.982 54.867793) (width 0.2) (layer "F.Cu") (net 3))
 (segment (start 108.384207 52.27) (end 104.555 52.27) (width 0.2) (layer "F.Cu") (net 3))
 (segment (start 109.427401 71.05) (end 110.982 69.495401) (width 0.2) (layer "F.Cu") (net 3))
 (segment (start 152.02 66.9375) (end 155.1375 66.9375) (width 0.2) (layer "F.Cu") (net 25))
 (segment (start 145.96 75) (end 144.809 76.151) (width 0.2) (layer "F.Cu") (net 20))
 (segment (start 140.315 72.56924) (end 140.315 66.81) (width 0.2) (layer "F.Cu") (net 20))
 (segment (start 145.96 69.9775) (end 145.96 75) (width 0.2) (layer "F.Cu") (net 20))
 (segment (start 142.2075 66.9375) (end 142.15 66.88) (width 0.2) (layer "F.Cu") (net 20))
 (segment (start 142.92 66.9375) (end 145.96 69.9775) (width 0.2) (layer "F.Cu") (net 20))
 (segment (start 142.94324 76.151) (end 142.269 75.47676) (width 0.2) (layer "F.Cu") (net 20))
 (segment (start 142.269 74.52324) (end 140.315 72.56924) (width 0.2) (layer "F.Cu") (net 20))
 (segment (start 142.15 66.88) (end 142.15 66.81) (width 0.2) (layer "F.Cu") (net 20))
 (segment (start 142.269 75.47676) (end 142.269 74.52324) (width 0.2) (layer "F.Cu") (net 20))
 (segment (start 144.809 76.151) (end 142.94324 76.151) (width 0.2) (layer "F.Cu") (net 20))
 (segment (start 142.7925 66.81) (end 142.15 66.81) (width 0.2) (layer "F.Cu") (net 20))
 (segment (start 152.7975 59.5125) (end 155.2 59.5125) (width 0.2) (layer "F.Cu") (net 13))
 (segment (start 140.315 64.27) (end 139.214 63.169) (width 0.2) (layer "F.Cu") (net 21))
 (segment (start 139.214 61.27395) (end 140.19695 60.291) (width 0.2) (layer "F.Cu") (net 21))
 (segment (start 139.85895 60.629) (end 140.77105 60.629) (width 0.2) (layer "F.Cu") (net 21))
 (segment (start 140.19695 60.291) (end 142.4265 60.291) (width 0.2) (layer "F.Cu") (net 21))
 (segment (start 139.214 63.169) (end 139.214 61.27395) (width 0.2) (layer "F.Cu") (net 21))
 (segment (start 148.5 68.35795) (end 148.5 75) (width 0.2) (layer "F.Cu") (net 21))
 (segment (start 142.4265 60.291) (end 143.17 59.5475) (width 0.2) (layer "F.Cu") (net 21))
 (segment (start 140.77105 60.629) (end 148.5 68.35795) (width 0.2) (layer "F.Cu") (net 21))
 (segment (start 139.214 61.27395) (end 139.85895 60.629) (width 0.2) (layer "F.Cu") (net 21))
 (segment (start 130.5 61.55) (end 132.515 61.55) (width 0.2) (layer "F.Cu") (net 15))
 (segment (start 121.43 58.1) (end 121.43 61.52) (width 0.2) (layer "F.Cu") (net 14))
 (segment (start 113.694213 54.7) (end 119.551 60.556787) (width 0.2) (layer "F.Cu") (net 22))
 (segment (start 119.551 60.556787) (end 119.551 61.971) (width 0.2) (layer "F.Cu") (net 22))
 (segment (start 119.551 61.971) (end 121.85 64.27) (width 0.2) (layer "F.Cu") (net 22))
 (segment (start 121.85 64.27) (end 132.695 64.27) (width 0.2) (layer "F.Cu") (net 22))
 (segment (start 112.28 54.7) (end 113.694213 54.7) (width 0.2) (layer "F.Cu") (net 22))
 (segment (start 141.749 73.329) (end 143.42 75) (width 0.2) (layer "F.Cu") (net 19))
 (segment (start 140.315 61.73) (end 141.749 63.164) (width 0.2) (layer "F.Cu") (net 19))
 (segment (start 141.749 63.164) (end 141.749 73.329) (width 0.2) (layer "F.Cu") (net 19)))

